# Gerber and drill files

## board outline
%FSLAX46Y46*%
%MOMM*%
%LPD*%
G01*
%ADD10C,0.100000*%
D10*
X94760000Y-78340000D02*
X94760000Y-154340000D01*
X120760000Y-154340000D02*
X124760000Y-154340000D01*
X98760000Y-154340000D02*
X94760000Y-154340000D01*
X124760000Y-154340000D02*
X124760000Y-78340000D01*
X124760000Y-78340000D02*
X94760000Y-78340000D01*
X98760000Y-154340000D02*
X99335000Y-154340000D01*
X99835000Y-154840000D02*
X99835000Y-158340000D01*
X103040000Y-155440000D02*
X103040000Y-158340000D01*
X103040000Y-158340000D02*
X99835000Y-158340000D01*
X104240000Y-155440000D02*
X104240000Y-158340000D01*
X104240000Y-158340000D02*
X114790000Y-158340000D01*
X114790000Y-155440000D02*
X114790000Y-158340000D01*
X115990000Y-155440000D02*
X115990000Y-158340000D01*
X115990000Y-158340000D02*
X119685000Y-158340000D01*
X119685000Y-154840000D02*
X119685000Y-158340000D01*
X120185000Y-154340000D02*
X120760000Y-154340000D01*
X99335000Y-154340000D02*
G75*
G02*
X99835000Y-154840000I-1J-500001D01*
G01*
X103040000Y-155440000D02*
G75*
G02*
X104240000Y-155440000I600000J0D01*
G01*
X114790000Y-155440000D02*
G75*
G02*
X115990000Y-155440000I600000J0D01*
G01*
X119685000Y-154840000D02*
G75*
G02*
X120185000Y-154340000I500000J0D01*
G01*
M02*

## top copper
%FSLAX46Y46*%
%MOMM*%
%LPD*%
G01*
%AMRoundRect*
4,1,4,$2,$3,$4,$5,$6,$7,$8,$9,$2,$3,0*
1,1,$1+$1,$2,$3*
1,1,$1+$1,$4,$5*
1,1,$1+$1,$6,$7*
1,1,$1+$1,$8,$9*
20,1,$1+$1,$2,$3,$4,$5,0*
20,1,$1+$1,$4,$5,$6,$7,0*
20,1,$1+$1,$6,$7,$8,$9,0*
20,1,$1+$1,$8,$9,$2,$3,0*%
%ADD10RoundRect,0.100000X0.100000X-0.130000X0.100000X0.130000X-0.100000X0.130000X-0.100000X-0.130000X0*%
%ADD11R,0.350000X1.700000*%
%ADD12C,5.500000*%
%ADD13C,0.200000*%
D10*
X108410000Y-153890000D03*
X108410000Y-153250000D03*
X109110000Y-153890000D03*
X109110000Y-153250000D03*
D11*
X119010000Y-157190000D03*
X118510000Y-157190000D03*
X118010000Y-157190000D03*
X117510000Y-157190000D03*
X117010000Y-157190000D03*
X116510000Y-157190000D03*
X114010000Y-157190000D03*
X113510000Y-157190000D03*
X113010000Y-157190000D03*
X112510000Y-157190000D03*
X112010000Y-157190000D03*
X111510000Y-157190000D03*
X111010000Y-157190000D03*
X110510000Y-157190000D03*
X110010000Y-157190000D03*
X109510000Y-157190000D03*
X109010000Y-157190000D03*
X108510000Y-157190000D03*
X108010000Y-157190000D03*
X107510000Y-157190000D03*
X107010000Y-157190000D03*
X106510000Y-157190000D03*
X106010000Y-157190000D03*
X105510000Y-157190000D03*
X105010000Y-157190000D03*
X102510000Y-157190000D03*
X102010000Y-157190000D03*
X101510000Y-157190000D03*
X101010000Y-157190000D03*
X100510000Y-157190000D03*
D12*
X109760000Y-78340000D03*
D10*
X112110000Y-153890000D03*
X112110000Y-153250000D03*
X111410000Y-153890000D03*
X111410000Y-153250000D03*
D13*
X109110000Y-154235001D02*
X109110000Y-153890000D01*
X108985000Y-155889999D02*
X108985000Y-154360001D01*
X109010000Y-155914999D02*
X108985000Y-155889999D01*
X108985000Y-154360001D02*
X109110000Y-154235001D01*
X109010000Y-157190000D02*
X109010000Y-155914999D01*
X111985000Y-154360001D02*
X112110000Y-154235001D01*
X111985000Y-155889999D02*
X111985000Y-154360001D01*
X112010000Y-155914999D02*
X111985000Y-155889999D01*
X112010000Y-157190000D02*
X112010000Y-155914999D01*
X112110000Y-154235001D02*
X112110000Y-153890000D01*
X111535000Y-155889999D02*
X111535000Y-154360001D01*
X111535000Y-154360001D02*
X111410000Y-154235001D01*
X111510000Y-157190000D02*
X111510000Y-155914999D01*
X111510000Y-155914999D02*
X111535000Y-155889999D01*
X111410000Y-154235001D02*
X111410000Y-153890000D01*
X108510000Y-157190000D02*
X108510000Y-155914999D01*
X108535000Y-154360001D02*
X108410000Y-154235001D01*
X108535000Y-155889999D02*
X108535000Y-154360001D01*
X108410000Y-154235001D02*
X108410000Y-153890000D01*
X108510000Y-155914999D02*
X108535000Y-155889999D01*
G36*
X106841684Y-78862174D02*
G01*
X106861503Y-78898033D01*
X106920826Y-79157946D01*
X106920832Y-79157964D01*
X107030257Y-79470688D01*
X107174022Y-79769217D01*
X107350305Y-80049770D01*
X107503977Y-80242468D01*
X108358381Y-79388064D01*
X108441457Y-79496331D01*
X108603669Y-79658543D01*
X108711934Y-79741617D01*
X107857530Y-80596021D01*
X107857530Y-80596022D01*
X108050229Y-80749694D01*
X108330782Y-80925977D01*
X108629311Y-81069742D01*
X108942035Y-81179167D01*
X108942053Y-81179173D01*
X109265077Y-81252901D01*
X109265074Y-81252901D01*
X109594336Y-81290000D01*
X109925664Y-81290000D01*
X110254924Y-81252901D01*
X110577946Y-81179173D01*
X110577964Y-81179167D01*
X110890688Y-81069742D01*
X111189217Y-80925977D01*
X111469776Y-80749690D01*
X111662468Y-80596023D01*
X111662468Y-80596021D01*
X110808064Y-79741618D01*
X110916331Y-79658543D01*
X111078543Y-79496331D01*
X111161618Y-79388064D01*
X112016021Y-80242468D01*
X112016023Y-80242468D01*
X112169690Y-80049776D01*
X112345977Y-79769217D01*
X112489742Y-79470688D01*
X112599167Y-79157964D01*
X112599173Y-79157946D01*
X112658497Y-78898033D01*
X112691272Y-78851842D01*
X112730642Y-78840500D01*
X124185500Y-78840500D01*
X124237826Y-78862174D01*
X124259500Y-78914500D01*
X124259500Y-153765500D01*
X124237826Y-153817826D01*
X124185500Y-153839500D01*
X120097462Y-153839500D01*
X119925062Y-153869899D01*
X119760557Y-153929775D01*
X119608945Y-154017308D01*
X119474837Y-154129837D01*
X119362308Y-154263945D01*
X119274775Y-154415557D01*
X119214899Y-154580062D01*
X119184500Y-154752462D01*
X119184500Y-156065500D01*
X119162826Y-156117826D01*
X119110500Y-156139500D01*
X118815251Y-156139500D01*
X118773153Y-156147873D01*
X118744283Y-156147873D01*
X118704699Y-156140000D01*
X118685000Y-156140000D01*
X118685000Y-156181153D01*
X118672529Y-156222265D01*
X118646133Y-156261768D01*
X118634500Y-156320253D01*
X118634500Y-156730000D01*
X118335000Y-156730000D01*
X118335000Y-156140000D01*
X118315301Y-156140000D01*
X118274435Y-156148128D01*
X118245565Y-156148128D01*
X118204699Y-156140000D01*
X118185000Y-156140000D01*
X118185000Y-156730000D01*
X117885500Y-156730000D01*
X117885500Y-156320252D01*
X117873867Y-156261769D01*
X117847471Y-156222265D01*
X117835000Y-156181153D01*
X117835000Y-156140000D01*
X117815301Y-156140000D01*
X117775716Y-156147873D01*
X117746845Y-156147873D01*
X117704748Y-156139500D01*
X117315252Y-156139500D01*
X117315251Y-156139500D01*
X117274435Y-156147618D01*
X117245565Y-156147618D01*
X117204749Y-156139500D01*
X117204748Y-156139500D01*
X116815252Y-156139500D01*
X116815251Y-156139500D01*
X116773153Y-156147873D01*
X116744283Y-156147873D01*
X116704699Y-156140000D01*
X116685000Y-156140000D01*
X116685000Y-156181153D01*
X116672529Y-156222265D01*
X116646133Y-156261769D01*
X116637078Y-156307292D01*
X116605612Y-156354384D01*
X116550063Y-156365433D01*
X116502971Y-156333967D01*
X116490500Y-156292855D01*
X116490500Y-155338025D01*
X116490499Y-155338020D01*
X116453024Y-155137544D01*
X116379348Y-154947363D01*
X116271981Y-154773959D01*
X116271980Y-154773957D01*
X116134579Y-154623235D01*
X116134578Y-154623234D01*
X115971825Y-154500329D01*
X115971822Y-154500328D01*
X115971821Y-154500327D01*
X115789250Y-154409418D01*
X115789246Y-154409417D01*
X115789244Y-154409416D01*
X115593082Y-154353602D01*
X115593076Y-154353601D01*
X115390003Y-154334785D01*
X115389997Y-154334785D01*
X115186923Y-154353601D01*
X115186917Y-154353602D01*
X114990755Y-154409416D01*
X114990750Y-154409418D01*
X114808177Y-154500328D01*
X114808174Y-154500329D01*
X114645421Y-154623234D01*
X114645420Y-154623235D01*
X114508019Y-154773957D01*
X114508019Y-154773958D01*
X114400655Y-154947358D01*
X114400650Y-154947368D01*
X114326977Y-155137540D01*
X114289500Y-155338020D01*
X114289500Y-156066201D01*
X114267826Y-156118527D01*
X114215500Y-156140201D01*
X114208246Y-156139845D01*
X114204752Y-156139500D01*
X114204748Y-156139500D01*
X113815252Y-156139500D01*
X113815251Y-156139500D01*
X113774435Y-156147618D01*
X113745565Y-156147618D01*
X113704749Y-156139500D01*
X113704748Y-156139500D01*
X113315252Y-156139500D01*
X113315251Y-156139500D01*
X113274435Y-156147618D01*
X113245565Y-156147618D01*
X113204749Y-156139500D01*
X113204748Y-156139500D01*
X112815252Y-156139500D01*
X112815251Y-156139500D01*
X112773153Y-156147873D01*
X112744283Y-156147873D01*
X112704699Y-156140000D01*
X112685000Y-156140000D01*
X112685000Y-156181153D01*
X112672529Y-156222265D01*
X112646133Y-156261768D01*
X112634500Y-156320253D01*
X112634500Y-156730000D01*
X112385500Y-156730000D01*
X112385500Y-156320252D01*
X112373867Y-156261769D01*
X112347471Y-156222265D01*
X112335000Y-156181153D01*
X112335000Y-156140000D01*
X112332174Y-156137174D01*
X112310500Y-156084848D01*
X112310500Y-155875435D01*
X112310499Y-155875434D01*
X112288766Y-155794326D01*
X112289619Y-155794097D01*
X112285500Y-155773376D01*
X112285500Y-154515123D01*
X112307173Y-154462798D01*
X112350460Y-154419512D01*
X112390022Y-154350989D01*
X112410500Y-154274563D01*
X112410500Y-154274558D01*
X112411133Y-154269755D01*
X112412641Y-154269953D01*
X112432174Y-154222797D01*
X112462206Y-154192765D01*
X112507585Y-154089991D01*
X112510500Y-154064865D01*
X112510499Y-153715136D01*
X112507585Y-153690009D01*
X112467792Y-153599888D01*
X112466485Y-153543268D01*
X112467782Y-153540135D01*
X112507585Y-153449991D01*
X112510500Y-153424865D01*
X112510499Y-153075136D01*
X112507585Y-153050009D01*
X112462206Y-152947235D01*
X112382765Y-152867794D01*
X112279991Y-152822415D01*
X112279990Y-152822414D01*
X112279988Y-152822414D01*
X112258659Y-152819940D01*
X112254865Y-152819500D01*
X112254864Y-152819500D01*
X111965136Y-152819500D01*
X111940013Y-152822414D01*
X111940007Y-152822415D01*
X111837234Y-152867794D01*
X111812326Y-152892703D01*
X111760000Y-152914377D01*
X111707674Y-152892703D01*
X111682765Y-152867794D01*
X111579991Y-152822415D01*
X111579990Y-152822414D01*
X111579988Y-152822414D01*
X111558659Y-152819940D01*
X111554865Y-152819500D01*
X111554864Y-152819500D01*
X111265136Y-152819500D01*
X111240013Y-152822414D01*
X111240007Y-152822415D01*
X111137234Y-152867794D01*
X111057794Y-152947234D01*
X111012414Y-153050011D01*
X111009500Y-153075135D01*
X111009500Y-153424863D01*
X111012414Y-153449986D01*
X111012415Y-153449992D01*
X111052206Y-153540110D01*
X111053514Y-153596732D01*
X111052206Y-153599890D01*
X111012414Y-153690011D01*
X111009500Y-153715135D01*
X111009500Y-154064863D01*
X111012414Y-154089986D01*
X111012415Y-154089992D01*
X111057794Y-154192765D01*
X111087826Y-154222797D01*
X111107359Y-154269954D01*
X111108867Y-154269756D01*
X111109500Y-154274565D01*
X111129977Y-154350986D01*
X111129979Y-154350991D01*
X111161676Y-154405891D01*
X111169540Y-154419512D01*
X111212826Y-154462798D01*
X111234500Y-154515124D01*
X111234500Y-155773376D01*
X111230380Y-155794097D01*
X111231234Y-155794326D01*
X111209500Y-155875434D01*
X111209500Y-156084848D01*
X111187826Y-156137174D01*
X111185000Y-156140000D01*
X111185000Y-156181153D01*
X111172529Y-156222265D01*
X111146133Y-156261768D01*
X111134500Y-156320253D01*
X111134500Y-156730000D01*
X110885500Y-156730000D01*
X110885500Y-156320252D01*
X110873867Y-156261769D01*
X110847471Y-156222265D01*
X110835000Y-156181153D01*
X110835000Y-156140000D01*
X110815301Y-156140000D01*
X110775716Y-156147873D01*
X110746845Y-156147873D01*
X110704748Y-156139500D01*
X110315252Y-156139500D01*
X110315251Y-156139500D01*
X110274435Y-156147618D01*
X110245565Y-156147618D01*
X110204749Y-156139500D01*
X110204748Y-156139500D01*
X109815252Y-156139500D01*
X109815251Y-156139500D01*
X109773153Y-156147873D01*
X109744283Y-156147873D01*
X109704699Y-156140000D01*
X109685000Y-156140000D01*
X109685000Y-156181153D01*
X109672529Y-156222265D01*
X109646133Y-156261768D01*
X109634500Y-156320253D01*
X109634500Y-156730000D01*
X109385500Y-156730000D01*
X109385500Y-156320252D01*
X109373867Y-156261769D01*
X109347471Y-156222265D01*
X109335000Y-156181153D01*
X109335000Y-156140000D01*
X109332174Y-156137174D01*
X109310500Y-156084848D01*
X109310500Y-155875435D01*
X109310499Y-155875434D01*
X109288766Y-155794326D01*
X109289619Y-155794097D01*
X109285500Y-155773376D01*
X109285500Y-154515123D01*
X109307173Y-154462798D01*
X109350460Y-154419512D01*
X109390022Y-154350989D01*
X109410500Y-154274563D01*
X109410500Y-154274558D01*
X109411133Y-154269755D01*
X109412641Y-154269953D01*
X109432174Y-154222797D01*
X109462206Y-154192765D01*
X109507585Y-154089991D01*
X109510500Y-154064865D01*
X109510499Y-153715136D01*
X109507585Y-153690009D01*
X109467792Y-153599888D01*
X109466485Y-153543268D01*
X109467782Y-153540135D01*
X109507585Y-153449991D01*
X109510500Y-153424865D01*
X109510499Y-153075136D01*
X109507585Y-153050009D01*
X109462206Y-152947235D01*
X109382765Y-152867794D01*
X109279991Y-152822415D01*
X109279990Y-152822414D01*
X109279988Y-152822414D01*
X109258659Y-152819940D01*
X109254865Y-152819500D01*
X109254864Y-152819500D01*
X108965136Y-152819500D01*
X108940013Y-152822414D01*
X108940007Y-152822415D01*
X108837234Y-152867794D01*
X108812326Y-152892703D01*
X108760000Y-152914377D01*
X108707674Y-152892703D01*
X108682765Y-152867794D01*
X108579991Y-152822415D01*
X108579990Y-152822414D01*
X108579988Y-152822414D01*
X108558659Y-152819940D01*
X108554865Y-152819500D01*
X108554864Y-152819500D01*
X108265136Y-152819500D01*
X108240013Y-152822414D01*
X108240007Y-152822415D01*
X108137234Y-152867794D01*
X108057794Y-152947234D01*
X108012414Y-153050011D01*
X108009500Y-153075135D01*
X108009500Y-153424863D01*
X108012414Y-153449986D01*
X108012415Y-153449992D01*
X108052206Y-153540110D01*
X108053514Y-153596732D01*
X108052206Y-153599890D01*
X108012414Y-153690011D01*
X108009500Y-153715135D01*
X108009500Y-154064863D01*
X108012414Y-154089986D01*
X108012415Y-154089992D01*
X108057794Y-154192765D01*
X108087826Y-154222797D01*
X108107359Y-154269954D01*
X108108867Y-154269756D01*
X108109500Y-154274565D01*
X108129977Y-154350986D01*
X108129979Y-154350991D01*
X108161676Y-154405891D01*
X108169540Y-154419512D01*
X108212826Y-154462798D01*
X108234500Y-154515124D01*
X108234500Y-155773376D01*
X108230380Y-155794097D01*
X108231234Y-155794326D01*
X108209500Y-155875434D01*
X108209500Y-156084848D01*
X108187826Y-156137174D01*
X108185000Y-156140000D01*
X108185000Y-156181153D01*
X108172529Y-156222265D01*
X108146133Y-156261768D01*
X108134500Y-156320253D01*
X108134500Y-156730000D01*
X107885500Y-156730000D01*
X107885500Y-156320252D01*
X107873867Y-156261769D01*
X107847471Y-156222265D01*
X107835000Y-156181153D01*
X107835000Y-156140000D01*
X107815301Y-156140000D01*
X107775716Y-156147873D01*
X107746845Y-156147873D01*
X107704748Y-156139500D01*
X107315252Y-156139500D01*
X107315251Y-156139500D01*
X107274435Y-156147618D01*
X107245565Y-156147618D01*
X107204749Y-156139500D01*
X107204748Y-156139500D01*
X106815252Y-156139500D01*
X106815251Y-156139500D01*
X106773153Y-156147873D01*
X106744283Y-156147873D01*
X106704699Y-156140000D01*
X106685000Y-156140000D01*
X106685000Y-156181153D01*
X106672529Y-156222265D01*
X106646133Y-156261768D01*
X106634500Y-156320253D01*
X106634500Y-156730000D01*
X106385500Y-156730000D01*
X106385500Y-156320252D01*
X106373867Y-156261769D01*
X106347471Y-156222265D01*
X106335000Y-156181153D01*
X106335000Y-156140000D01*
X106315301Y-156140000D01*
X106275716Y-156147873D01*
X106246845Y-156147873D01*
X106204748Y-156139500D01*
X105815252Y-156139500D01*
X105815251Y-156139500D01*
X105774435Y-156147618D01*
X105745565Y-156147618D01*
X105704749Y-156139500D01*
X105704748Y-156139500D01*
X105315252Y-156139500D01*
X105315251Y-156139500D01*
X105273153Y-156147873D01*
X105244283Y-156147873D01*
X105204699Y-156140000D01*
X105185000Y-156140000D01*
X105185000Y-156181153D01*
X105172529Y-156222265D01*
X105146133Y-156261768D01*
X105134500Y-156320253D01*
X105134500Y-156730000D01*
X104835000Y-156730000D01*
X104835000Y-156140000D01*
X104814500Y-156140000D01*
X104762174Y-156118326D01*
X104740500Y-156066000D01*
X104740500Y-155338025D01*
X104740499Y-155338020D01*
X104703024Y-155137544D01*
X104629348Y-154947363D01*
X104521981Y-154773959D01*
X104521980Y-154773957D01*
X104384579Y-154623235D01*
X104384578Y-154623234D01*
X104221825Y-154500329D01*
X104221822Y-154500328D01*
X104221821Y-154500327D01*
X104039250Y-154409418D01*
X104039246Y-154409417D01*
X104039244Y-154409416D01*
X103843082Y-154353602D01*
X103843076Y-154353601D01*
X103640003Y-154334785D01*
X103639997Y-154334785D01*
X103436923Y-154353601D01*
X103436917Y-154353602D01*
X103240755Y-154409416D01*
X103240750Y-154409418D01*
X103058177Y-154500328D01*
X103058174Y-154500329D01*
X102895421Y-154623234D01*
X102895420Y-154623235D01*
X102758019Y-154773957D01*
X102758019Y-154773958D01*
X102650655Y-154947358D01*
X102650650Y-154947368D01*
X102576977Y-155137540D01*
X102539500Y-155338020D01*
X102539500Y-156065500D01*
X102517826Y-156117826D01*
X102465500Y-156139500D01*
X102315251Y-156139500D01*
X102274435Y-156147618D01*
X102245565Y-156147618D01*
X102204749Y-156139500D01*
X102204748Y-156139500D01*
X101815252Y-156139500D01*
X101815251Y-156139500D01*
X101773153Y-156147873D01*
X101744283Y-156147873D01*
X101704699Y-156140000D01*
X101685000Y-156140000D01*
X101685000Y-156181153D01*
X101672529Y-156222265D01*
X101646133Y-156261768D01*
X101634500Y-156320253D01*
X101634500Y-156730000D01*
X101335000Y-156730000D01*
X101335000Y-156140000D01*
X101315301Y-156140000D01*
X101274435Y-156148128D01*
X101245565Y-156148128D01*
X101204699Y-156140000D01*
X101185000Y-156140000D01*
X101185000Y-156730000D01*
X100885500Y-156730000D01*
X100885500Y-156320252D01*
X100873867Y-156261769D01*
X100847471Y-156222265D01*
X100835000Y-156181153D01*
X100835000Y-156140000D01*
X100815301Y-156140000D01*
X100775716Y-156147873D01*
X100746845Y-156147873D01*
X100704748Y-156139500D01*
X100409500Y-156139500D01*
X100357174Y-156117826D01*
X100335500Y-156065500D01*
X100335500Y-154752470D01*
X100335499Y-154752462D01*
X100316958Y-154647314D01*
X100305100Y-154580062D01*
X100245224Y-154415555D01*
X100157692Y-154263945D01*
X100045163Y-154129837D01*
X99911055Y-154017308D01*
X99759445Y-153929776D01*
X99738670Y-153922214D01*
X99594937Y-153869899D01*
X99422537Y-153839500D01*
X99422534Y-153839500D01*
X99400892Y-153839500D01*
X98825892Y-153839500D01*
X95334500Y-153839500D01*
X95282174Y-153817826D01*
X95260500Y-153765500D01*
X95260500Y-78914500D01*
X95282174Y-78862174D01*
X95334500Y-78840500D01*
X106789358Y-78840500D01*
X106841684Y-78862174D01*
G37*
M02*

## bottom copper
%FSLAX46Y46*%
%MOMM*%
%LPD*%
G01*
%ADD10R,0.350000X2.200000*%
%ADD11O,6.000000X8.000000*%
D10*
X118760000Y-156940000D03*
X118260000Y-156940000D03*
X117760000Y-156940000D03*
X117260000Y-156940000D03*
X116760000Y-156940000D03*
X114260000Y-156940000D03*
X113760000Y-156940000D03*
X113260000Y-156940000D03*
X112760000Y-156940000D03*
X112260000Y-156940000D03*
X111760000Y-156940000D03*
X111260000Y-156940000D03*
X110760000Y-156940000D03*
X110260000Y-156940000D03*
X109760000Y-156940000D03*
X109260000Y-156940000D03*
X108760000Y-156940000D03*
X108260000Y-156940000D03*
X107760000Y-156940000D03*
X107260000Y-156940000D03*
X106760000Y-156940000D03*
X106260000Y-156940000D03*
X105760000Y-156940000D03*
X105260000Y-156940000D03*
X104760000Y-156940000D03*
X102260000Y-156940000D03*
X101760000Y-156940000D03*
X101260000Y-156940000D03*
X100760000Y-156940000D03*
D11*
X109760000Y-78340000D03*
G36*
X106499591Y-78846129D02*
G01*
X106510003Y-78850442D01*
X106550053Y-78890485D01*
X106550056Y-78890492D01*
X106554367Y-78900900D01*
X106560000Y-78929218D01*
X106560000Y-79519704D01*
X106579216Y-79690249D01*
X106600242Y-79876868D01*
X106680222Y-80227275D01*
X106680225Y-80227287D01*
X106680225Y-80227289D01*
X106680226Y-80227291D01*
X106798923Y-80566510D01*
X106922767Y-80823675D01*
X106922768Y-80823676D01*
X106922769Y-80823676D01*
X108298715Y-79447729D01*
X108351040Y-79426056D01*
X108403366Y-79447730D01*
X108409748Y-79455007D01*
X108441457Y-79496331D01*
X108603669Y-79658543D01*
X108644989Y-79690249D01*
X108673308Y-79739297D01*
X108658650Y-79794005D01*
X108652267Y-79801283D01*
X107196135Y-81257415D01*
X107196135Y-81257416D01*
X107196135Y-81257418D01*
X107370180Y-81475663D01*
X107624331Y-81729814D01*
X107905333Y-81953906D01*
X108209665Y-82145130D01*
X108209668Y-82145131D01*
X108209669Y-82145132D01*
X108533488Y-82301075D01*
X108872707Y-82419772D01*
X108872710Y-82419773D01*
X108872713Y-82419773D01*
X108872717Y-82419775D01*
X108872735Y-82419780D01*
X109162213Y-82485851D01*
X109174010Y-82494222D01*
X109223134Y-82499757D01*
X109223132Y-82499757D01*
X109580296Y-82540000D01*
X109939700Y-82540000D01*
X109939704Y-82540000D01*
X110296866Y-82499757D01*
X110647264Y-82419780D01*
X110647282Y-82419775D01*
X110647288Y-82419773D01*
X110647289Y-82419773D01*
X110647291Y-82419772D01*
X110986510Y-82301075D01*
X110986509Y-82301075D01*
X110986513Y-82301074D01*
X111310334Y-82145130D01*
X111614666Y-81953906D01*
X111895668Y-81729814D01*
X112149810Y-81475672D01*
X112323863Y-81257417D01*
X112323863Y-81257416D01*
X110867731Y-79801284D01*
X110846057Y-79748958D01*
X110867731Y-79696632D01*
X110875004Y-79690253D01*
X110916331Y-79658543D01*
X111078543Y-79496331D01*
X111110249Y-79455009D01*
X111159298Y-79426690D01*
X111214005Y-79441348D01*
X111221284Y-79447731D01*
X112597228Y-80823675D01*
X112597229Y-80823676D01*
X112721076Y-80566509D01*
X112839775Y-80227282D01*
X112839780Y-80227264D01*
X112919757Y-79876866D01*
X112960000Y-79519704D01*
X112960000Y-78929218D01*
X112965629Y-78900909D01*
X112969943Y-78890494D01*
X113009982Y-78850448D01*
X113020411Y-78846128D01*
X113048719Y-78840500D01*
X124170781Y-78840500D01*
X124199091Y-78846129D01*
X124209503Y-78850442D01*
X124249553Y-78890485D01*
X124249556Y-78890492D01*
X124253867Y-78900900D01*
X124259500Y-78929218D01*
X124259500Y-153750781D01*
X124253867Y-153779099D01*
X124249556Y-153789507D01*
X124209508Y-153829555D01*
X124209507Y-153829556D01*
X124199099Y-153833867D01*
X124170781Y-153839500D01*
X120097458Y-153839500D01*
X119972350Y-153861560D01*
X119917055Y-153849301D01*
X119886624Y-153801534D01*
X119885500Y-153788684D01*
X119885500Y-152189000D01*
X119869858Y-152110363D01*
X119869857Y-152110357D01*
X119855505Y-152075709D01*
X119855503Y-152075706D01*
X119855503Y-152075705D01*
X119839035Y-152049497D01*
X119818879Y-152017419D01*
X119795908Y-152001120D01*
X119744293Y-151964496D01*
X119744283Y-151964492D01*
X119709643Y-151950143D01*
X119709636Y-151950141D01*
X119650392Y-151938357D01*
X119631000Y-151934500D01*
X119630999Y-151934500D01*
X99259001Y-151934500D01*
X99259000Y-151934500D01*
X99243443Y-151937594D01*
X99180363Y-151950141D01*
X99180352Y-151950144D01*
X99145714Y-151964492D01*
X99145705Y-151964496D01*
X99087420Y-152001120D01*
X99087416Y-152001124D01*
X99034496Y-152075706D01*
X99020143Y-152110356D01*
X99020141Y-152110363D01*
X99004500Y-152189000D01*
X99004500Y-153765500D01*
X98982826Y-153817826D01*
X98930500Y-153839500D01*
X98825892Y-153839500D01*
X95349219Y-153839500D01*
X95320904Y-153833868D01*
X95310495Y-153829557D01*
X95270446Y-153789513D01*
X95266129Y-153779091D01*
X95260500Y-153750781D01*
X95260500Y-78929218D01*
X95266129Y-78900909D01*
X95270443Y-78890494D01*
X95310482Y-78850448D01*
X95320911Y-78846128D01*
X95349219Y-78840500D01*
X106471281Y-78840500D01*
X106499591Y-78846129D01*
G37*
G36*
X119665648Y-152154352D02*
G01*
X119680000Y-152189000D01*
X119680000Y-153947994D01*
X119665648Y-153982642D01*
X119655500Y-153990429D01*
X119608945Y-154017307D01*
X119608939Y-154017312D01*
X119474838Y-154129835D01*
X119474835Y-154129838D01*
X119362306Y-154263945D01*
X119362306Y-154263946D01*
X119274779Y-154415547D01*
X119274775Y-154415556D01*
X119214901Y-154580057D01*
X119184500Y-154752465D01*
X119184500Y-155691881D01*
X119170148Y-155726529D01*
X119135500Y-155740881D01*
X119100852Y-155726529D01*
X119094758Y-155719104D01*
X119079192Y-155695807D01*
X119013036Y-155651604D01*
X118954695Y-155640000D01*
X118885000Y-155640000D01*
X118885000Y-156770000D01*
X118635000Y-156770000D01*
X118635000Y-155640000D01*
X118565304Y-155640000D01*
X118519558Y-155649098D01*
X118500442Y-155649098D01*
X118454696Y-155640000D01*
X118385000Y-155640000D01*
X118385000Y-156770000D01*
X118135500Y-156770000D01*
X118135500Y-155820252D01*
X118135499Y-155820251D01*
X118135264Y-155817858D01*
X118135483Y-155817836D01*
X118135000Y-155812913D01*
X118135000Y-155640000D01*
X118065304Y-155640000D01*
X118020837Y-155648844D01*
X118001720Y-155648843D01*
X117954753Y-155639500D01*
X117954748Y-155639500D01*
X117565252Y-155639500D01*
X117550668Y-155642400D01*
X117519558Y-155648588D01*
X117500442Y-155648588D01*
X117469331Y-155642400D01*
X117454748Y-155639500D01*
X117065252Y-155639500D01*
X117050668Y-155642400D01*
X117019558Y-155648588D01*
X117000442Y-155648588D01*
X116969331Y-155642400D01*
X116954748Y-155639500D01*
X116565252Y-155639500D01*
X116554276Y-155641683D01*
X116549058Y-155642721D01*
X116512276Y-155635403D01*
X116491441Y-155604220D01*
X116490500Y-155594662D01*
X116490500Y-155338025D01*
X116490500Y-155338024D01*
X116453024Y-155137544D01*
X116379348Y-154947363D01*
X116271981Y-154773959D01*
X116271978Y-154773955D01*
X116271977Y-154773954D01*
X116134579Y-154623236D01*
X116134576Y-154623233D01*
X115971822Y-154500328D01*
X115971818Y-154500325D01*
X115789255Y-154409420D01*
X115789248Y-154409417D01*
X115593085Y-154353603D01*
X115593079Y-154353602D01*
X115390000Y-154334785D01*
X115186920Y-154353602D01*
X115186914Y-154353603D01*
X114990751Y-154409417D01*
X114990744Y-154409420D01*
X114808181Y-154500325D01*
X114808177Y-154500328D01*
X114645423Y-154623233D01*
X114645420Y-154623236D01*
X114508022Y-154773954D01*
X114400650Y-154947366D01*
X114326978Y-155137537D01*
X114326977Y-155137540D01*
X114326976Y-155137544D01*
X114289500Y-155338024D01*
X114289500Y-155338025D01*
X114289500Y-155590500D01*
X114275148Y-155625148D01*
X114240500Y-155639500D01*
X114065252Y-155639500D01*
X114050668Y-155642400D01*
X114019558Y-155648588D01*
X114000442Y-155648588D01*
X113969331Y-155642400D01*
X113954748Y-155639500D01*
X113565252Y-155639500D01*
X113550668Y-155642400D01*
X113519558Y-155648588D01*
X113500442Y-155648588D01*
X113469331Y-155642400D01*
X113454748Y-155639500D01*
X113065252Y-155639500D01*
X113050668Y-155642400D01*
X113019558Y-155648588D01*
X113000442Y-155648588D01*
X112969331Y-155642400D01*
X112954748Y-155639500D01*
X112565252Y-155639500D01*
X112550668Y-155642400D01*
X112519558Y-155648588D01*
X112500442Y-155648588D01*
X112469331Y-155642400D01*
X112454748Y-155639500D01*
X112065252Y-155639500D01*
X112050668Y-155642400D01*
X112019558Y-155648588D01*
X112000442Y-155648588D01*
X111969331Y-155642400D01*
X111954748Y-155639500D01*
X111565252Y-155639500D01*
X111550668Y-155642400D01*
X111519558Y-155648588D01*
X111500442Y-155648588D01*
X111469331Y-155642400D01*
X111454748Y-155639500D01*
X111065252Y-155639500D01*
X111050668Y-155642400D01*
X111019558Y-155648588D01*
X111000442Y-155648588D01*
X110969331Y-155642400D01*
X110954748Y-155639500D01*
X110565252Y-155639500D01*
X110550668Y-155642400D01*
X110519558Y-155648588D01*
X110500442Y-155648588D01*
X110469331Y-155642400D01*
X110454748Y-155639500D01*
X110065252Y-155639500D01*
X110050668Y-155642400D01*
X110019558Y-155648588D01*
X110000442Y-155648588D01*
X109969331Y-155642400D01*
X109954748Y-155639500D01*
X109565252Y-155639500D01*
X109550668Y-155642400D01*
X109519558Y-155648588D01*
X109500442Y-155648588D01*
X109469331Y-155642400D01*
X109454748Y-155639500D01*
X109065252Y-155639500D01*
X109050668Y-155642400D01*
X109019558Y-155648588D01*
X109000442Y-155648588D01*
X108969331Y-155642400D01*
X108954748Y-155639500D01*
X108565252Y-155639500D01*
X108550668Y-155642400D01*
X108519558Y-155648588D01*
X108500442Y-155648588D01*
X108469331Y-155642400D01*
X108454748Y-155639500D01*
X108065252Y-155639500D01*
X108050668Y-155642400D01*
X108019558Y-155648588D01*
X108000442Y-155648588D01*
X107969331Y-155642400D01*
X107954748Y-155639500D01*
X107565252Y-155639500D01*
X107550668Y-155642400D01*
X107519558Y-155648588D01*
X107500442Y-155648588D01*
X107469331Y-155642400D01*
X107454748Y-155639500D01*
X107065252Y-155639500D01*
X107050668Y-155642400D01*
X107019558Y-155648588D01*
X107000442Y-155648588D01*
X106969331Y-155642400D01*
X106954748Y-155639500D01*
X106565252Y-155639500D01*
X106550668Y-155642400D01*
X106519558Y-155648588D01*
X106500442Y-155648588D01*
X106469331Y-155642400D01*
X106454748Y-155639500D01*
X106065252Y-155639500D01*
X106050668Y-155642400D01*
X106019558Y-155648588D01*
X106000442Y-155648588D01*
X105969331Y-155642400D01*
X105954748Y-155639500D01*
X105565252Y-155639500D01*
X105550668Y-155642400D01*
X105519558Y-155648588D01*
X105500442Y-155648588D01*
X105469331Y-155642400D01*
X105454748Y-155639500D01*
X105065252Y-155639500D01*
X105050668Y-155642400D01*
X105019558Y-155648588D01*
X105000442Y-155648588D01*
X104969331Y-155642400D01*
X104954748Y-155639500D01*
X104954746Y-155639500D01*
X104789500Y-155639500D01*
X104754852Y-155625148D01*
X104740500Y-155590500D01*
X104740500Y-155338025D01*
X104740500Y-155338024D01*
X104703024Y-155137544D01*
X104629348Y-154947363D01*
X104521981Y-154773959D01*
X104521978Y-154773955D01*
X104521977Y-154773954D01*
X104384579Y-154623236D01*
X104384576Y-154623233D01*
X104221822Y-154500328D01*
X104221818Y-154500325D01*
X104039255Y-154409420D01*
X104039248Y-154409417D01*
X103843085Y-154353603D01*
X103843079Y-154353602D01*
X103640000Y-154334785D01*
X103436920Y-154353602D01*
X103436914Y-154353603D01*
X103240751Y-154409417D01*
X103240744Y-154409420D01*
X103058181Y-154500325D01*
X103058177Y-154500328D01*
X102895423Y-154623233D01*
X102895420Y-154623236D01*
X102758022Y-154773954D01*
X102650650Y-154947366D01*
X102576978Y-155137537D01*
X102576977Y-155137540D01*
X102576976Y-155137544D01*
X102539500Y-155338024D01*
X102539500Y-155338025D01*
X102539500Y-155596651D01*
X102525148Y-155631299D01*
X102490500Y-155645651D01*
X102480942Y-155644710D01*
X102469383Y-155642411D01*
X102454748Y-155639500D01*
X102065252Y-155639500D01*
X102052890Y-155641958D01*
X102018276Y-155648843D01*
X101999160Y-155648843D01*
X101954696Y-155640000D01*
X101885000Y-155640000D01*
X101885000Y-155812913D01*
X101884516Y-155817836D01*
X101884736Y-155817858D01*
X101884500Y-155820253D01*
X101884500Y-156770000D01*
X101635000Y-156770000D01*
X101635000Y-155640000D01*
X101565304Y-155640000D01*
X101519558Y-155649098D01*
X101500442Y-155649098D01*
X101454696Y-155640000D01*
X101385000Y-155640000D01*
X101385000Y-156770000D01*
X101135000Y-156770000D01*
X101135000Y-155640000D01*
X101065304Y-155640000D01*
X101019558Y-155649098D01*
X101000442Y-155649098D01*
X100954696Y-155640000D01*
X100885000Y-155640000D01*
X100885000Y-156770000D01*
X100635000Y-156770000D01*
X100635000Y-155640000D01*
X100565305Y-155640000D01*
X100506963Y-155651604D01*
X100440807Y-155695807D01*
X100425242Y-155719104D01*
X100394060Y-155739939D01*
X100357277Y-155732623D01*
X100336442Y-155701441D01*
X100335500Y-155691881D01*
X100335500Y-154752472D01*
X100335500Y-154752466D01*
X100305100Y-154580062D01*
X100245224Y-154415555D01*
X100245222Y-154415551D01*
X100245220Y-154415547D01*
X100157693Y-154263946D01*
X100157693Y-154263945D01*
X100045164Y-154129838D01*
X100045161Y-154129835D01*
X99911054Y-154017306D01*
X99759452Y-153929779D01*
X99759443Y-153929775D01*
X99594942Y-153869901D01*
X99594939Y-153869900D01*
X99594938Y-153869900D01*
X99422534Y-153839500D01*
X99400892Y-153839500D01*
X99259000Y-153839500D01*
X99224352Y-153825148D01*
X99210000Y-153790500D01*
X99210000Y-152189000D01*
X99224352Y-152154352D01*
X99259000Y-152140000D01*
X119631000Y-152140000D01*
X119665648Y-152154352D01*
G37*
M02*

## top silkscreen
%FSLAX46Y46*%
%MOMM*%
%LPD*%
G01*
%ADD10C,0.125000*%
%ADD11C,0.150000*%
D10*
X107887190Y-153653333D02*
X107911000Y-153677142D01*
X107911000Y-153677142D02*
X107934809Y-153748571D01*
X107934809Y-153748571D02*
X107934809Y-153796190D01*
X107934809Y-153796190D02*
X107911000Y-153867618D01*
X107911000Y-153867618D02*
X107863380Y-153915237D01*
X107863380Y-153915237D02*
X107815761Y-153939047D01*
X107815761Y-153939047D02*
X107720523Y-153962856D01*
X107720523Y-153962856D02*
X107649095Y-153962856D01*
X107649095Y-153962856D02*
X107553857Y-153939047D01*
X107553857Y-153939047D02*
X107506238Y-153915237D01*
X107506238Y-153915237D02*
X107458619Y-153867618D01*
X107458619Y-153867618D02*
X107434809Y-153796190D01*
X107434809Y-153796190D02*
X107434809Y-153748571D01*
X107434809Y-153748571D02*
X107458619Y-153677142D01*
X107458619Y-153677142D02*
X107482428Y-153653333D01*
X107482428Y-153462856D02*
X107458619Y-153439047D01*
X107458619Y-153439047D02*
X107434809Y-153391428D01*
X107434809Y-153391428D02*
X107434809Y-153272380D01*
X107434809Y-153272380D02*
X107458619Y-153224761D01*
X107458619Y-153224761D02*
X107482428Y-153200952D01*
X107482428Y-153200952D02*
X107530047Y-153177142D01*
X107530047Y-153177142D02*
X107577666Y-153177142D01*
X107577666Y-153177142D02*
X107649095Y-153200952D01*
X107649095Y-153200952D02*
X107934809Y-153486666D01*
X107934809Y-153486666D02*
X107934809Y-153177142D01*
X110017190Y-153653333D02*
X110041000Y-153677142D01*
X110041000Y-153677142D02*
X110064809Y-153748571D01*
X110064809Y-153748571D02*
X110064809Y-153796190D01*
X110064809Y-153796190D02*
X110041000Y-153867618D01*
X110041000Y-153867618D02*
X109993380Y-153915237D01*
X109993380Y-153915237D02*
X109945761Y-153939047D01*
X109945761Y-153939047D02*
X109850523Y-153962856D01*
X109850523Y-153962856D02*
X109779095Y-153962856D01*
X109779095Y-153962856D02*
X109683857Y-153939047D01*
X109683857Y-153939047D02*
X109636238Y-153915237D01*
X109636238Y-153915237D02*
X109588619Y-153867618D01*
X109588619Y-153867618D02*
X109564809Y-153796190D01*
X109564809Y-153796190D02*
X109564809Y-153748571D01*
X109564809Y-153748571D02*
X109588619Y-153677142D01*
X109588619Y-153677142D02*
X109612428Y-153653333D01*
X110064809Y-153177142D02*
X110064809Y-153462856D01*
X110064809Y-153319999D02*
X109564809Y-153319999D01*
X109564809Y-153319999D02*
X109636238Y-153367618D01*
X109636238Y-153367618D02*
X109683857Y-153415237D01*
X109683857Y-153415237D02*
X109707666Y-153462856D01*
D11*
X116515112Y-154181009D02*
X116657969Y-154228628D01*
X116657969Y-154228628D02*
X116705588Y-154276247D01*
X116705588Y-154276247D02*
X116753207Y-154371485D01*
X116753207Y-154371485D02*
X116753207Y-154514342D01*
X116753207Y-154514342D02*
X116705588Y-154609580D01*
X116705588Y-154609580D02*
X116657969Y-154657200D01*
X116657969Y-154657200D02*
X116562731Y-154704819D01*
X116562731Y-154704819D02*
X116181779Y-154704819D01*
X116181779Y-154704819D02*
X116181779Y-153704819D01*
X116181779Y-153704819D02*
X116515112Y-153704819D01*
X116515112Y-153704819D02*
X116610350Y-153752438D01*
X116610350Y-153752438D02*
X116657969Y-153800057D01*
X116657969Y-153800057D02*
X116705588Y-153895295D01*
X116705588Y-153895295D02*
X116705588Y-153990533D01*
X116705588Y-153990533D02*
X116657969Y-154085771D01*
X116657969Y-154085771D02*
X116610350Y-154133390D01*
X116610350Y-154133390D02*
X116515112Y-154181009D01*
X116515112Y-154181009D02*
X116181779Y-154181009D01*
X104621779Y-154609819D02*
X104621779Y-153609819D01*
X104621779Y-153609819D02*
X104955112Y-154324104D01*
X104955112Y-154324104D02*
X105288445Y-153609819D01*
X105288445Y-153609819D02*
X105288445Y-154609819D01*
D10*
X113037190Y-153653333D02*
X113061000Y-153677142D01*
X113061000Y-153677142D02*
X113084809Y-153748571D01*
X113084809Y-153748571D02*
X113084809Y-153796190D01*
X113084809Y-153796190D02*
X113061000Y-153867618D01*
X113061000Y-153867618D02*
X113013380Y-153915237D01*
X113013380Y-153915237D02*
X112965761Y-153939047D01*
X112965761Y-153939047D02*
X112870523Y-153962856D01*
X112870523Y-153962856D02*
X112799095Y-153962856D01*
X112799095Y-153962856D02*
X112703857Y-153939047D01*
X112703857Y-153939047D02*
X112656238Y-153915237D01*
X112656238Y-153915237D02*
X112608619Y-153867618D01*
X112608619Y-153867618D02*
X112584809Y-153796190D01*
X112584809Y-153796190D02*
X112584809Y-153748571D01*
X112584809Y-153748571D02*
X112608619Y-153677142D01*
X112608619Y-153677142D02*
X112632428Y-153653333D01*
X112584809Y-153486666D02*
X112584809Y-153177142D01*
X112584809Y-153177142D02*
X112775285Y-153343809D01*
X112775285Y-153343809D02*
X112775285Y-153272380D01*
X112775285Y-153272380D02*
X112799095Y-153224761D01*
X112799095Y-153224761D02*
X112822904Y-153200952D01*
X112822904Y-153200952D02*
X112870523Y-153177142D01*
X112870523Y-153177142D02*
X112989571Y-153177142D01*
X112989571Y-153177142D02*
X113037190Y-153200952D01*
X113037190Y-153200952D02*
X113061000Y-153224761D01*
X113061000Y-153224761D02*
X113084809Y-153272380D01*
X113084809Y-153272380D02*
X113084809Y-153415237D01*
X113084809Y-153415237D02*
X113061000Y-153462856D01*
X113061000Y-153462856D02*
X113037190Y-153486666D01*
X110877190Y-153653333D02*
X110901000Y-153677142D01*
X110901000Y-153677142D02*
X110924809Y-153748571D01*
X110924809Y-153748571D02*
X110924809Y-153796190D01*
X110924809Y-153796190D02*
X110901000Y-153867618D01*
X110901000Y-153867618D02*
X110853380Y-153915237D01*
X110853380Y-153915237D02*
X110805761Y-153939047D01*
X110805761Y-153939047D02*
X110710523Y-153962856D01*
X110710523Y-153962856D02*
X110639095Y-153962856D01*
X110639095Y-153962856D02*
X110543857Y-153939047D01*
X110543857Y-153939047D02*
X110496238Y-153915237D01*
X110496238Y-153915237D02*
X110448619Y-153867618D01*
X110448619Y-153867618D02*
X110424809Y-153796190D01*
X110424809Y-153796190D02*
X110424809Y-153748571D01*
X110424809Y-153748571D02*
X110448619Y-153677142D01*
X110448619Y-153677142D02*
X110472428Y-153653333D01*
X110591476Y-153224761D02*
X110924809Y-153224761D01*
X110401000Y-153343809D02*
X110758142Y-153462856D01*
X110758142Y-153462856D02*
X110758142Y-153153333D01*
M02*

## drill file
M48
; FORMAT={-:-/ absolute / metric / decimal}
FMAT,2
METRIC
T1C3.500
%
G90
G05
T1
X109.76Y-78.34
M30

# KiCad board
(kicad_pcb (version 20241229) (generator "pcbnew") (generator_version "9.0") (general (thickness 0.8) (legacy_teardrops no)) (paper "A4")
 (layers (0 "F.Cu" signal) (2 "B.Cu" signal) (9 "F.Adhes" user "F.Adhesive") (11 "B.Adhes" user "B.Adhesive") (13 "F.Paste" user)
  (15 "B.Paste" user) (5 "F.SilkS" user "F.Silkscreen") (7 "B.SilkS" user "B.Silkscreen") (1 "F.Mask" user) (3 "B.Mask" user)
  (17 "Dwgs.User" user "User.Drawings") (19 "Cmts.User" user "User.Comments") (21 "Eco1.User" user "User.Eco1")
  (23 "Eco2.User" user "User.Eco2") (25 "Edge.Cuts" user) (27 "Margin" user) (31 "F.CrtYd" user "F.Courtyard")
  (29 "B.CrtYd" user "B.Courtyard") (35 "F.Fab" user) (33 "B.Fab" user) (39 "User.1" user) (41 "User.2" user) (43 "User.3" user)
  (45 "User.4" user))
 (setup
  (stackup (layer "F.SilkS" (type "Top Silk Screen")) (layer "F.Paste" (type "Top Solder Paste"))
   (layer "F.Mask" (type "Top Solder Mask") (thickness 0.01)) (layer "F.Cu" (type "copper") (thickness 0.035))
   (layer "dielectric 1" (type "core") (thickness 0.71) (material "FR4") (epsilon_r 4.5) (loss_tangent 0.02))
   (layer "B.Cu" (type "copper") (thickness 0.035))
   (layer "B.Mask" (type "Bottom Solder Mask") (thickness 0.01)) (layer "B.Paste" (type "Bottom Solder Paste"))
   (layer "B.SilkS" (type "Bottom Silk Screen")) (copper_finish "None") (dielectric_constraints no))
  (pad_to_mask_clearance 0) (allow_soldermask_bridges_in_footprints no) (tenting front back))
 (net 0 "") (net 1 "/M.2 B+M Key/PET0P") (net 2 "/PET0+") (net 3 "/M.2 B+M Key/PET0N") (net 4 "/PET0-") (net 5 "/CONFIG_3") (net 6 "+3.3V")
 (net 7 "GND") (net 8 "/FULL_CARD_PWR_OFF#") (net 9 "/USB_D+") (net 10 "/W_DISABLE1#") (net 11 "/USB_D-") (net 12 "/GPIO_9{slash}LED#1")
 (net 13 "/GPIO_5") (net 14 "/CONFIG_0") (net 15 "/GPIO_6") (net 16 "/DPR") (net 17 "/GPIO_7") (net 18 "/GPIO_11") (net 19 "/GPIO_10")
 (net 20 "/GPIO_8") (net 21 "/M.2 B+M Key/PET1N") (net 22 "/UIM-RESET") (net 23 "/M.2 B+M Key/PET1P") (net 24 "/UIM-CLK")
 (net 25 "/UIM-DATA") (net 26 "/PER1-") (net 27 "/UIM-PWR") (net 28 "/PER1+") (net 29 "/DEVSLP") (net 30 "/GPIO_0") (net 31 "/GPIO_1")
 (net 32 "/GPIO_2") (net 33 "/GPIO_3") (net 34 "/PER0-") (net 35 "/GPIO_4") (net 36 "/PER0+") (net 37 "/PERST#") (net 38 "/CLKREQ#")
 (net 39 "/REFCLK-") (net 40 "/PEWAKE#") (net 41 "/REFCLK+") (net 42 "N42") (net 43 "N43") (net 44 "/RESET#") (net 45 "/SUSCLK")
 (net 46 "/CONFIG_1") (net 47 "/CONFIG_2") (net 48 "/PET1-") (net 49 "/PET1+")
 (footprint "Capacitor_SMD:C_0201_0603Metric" (layer "F.Cu") (at 108.41 153.57 90)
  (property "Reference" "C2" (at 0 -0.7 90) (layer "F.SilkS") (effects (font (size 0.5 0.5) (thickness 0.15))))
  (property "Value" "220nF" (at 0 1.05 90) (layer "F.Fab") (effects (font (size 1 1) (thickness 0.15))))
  (pad "" smd roundrect (at -0.345 0 90) (size 0.318 0.36) (layers "F.Paste") (roundrect_rratio 0.25))
  (pad "" smd roundrect (at 0.345 0 90) (size 0.318 0.36) (layers "F.Paste") (roundrect_rratio 0.25))
  (pad "1" smd roundrect (at -0.32 0 90) (size 0.46 0.4) (layers "F.Cu" "F.Mask") (roundrect_rratio 0.25) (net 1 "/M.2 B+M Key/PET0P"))
  (pad "2" smd roundrect (at 0.32 0 90) (size 0.46 0.4) (layers "F.Cu" "F.Mask") (roundrect_rratio 0.25) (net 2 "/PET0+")))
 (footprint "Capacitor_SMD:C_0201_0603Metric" (layer "F.Cu") (at 109.11 153.57 90)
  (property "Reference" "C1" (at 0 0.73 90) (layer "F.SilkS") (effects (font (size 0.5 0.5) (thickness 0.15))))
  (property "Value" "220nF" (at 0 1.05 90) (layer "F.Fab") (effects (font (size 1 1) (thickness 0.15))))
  (pad "" smd roundrect (at -0.345 0 90) (size 0.318 0.36) (layers "F.Paste") (roundrect_rratio 0.25))
  (pad "" smd roundrect (at 0.345 0 90) (size 0.318 0.36) (layers "F.Paste") (roundrect_rratio 0.25))
  (pad "1" smd roundrect (at -0.32 0 90) (size 0.46 0.4) (layers "F.Cu" "F.Mask") (roundrect_rratio 0.25) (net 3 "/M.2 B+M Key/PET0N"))
  (pad "2" smd roundrect (at 0.32 0 90) (size 0.46 0.4) (layers "F.Cu" "F.Mask") (roundrect_rratio 0.25) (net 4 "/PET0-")))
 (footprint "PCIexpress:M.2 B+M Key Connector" (layer "F.Cu") (at 109.76 157.23)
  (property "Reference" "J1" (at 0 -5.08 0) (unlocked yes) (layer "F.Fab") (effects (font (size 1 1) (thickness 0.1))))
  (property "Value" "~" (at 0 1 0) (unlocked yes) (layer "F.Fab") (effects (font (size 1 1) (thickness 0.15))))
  (fp_line (start -11 -2.89) (end -10.425 -2.89) (stroke (width 0.1) (type default)) (layer "Edge.Cuts"))
  (fp_line (start -9.925 -2.39) (end -9.925 1.11) (stroke (width 0.1) (type default)) (layer "Edge.Cuts"))
  (fp_line (start -6.72 -1.79) (end -6.72 1.11) (stroke (width 0.1) (type default)) (layer "Edge.Cuts"))
  (fp_line (start -6.72 1.11) (end -9.925 1.11) (stroke (width 0.1) (type default)) (layer "Edge.Cuts"))
  (fp_line (start -5.52 -1.79) (end -5.52 1.11) (stroke (width 0.1) (type default)) (layer "Edge.Cuts"))
  (fp_line (start -5.52 1.11) (end 5.03 1.11) (stroke (width 0.1) (type default)) (layer "Edge.Cuts"))
  (fp_line (start 5.03 -1.79) (end 5.03 1.11) (stroke (width 0.1) (type default)) (layer "Edge.Cuts"))
  (fp_line (start 6.23 -1.79) (end 6.23 1.11) (stroke (width 0.1) (type default)) (layer "Edge.Cuts"))
  (fp_line (start 6.23 1.11) (end 9.925 1.11) (stroke (width 0.1) (type default)) (layer "Edge.Cuts"))
  (fp_line (start 9.925 -2.39) (end 9.925 1.11) (stroke (width 0.1) (type default)) (layer "Edge.Cuts"))
  (fp_line (start 10.425 -2.89) (end 11 -2.89) (stroke (width 0.1) (type default)) (layer "Edge.Cuts"))
  (fp_arc (start -10.425 -2.89) (mid -10.071447 -2.743553) (end -9.925 -2.39) (stroke (width 0.1) (type default)) (layer "Edge.Cuts"))
  (fp_arc (start -6.72 -1.79) (mid -6.12 -2.39) (end -5.52 -1.79) (stroke (width 0.1) (type default)) (layer "Edge.Cuts"))
  (fp_arc (start 5.03 -1.79) (mid 5.63 -2.39) (end 6.23 -1.79) (stroke (width 0.1) (type default)) (layer "Edge.Cuts"))
  (fp_arc (start 9.925 -2.39) (mid 10.071447 -2.743553) (end 10.425 -2.89) (stroke (width 0.1) (type default)) (layer "Edge.Cuts"))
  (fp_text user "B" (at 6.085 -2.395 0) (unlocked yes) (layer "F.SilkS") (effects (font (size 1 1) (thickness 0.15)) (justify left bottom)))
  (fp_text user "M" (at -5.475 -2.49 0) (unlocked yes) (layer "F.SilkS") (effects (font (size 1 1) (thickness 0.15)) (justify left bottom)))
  (pad "1" smd rect (at 9.25 -0.04 180) (size 0.35 1.7) (layers "F.Cu") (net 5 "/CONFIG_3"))
  (pad "2" smd rect (at 9 -0.29 180) (size 0.35 2.2) (layers "B.Cu") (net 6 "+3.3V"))
  (pad "3" smd rect (at 8.75 -0.04 180) (size 0.35 1.7) (layers "F.Cu") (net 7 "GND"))
  (pad "4" smd rect (at 8.5 -0.29 180) (size 0.35 2.2) (layers "B.Cu") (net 6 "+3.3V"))
  (pad "5" smd rect (at 8.25 -0.04 180) (size 0.35 1.7) (layers "F.Cu") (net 7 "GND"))
  (pad "6" smd rect (at 8 -0.29 180) (size 0.35 2.2) (layers "B.Cu") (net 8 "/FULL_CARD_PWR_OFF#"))
  (pad "7" smd rect (at 7.75 -0.04 180) (size 0.35 1.7) (layers "F.Cu") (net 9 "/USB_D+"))
  (pad "8" smd rect (at 7.5 -0.29 180) (size 0.35 2.2) (layers "B.Cu") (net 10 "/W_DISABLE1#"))
  (pad "9" smd rect (at 7.25 -0.04 180) (size 0.35 1.7) (layers "F.Cu") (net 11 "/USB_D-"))
  (pad "10" smd rect (at 7 -0.29 180) (size 0.35 2.2) (layers "B.Cu") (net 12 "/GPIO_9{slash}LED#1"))
  (pad "11" smd rect (at 6.75 -0.04 180) (size 0.35 1.7) (layers "F.Cu") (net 7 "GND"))
  (pad "20" smd rect (at 4.5 -0.29 180) (size 0.35 2.2) (layers "B.Cu") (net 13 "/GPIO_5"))
  (pad "21" smd rect (at 4.25 -0.04 180) (size 0.35 1.7) (layers "F.Cu") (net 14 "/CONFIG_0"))
  (pad "22" smd rect (at 4 -0.29 180) (size 0.35 2.2) (layers "B.Cu") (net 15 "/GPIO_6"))
  (pad "23" smd rect (at 3.75 -0.04 180) (size 0.35 1.7) (layers "F.Cu") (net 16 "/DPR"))
  (pad "24" smd rect (at 3.5 -0.29 180) (size 0.35 2.2) (layers "B.Cu") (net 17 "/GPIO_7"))
  (pad "25" smd rect (at 3.25 -0.04 180) (size 0.35 1.7) (layers "F.Cu") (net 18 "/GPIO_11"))
  (pad "26" smd rect (at 3 -0.29 180) (size 0.35 2.2) (layers "B.Cu") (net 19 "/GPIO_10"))
  (pad "27" smd rect (at 2.75 -0.04 180) (size 0.35 1.7) (layers "F.Cu") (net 7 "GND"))
  (pad "28" smd rect (at 2.5 -0.29 180) (size 0.35 2.2) (layers "B.Cu") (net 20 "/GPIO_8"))
  (pad "29" smd rect (at 2.25 -0.04 180) (size 0.35 1.7) (layers "F.Cu") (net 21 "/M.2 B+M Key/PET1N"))
  (pad "30" smd rect (at 2 -0.29 180) (size 0.35 2.2) (layers "B.Cu") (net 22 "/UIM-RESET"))
  (pad "31" smd rect (at 1.75 -0.04 180) (size 0.35 1.7) (layers "F.Cu") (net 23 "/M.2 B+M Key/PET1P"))
  (pad "32" smd rect (at 1.5 -0.29 180) (size 0.35 2.2) (layers "B.Cu") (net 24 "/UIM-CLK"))
  (pad "33" smd rect (at 1.25 -0.04 180) (size 0.35 1.7) (layers "F.Cu") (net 7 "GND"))
  (pad "34" smd rect (at 1 -0.29 180) (size 0.35 2.2) (layers "B.Cu") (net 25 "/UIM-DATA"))
  (pad "35" smd rect (at 0.75 -0.04 180) (size 0.35 1.7) (layers "F.Cu") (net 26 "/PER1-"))
  (pad "36" smd rect (at 0.5 -0.29 180) (size 0.35 2.2) (layers "B.Cu") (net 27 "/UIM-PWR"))
  (pad "37" smd rect (at 0.25 -0.04 180) (size 0.35 1.7) (layers "F.Cu") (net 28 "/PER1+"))
  (pad "38" smd rect (at 0 -0.29 180) (size 0.35 2.2) (layers "B.Cu") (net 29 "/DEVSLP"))
  (pad "39" smd rect (at -0.25 -0.04 180) (size 0.35 1.7) (layers "F.Cu") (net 7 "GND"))
  (pad "40" smd rect (at -0.5 -0.29 180) (size 0.35 2.2) (layers "B.Cu") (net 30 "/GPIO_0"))
  (pad "41" smd rect (at -0.75 -0.04 180) (size 0.35 1.7) (layers "F.Cu") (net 3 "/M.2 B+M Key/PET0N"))
  (pad "42" smd rect (at -1 -0.29 180) (size 0.35 2.2) (layers "B.Cu") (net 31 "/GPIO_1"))
  (pad "43" smd rect (at -1.25 -0.04 180) (size 0.35 1.7) (layers "F.Cu") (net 1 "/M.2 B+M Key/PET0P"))
  (pad "44" smd rect (at -1.5 -0.29 180) (size 0.35 2.2) (layers "B.Cu") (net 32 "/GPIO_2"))
  (pad "45" smd rect (at -1.75 -0.04 180) (size 0.35 1.7) (layers "F.Cu") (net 7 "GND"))
  (pad "46" smd rect (at -2 -0.29 180) (size 0.35 2.2) (layers "B.Cu") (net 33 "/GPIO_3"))
  (pad "47" smd rect (at -2.25 -0.04 180) (size 0.35 1.7) (layers "F.Cu") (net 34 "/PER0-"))
  (pad "48" smd rect (at -2.5 -0.29 180) (size 0.35 2.2) (layers "B.Cu") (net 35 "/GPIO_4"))
  (pad "49" smd rect (at -2.75 -0.04 180) (size 0.35 1.7) (layers "F.Cu") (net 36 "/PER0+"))
  (pad "50" smd rect (at -3 -0.29 180) (size 0.35 2.2) (layers "B.Cu") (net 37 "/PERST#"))
  (pad "51" smd rect (at -3.25 -0.04 180) (size 0.35 1.7) (layers "F.Cu") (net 7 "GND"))
  (pad "52" smd rect (at -3.5 -0.29 180) (size 0.35 2.2) (layers "B.Cu") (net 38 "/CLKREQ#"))
  (pad "53" smd rect (at -3.75 -0.04 180) (size 0.35 1.7) (layers "F.Cu") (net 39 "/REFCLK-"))
  (pad "54" smd rect (at -4 -0.29 180) (size 0.35 2.2) (layers "B.Cu") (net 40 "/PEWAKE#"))
  (pad "55" smd rect (at -4.25 -0.04 180) (size 0.35 1.7) (layers "F.Cu") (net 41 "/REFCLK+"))
  (pad "56" smd rect (at -4.5 -0.29 180) (size 0.35 2.2) (layers "B.Cu") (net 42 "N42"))
  (pad "57" smd rect (at -4.75 -0.04 180) (size 0.35 1.7) (layers "F.Cu") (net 7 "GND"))
  (pad "58" smd rect (at -5 -0.29 180) (size 0.35 2.2) (layers "B.Cu") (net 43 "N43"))
  (pad "67" smd rect (at -7.25 -0.04 180) (size 0.35 1.7) (layers "F.Cu") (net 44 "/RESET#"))
  (pad "68" smd rect (at -7.5 -0.29 180) (size 0.35 2.2) (layers "B.Cu") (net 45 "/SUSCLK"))
  (pad "69" smd rect (at -7.75 -0.04 180) (size 0.35 1.7) (layers "F.Cu") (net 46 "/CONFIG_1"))
  (pad "70" smd rect (at -8 -0.29 180) (size 0.35 2.2) (layers "B.Cu") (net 6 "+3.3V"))
  (pad "71" smd rect (at -8.25 -0.04 180) (size 0.35 1.7) (layers "F.Cu") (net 7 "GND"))
  (pad "72" smd rect (at -8.5 -0.29 180) (size 0.35 2.2) (layers "B.Cu") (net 6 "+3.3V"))
  (pad "73" smd rect (at -8.75 -0.04 180) (size 0.35 1.7) (layers "F.Cu") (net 7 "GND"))
  (pad "74" smd rect (at -9 -0.29 180) (size 0.35 2.2) (layers "B.Cu") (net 6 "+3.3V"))
  (pad "75" smd rect (at -9.25 -0.04 180) (size 0.35 1.7) (layers "F.Cu") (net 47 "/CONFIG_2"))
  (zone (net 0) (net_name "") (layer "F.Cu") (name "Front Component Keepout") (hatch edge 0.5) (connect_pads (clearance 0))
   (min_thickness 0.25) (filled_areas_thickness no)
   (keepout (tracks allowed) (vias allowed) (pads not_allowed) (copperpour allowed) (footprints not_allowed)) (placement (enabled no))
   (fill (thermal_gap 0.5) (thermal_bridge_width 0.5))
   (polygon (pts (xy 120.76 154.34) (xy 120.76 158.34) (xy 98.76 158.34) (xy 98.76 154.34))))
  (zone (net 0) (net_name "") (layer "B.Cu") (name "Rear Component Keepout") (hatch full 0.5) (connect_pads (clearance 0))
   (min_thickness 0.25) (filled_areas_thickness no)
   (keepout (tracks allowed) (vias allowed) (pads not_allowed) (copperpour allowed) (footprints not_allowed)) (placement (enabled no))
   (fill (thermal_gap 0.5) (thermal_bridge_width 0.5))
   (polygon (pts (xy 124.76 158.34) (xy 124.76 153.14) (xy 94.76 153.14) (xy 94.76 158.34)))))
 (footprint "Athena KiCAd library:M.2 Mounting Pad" (layer "F.Cu") (at 109.76 78.34)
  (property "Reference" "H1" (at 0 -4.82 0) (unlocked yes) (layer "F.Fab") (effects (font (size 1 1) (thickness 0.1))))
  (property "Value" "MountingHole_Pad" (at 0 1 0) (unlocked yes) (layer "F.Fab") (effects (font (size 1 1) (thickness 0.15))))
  (pad "1" thru_hole circle (at 0 0) (size 5.5 5.5) (drill 3.5) (layers "*.Cu" "*.Mask") (remove_unused_layers no) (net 7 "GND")
   (padstack (mode front_inner_back)
    (layer "Inner" (shape circle) (size 5.5 5.5) (zone_connect -1))
    (layer "B.Cu" (shape oval) (size 6 8) (thermal_bridge_angle 45) (zone_connect -1)))))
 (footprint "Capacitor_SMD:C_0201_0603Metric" (layer "F.Cu") (at 112.11 153.57 90)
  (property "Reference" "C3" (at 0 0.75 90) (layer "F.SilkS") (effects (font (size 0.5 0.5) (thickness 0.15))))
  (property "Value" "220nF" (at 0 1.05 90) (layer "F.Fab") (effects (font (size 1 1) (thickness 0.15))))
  (pad "" smd roundrect (at -0.345 0 90) (size 0.318 0.36) (layers "F.Paste") (roundrect_rratio 0.25))
  (pad "" smd roundrect (at 0.345 0 90) (size 0.318 0.36) (layers "F.Paste") (roundrect_rratio 0.25))
  (pad "1" smd roundrect (at -0.32 0 90) (size 0.46 0.4) (layers "F.Cu" "F.Mask") (roundrect_rratio 0.25) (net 21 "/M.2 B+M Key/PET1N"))
  (pad "2" smd roundrect (at 0.32 0 90) (size 0.46 0.4) (layers "F.Cu" "F.Mask") (roundrect_rratio 0.25) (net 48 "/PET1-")))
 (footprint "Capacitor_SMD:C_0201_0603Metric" (layer "F.Cu") (at 111.41 153.57 90)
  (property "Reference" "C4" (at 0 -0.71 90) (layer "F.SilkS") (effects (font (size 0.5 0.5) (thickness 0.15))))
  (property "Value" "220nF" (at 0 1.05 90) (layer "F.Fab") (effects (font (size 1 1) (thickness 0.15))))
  (pad "" smd roundrect (at -0.345 0 90) (size 0.318 0.36) (layers "F.Paste") (roundrect_rratio 0.25))
  (pad "" smd roundrect (at 0.345 0 90) (size 0.318 0.36) (layers "F.Paste") (roundrect_rratio 0.25))
  (pad "1" smd roundrect (at -0.32 0 90) (size 0.46 0.4) (layers "F.Cu" "F.Mask") (roundrect_rratio 0.25) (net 23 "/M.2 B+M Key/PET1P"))
  (pad "2" smd roundrect (at 0.32 0 90) (size 0.46 0.4) (layers "F.Cu" "F.Mask") (roundrect_rratio 0.25) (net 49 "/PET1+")))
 (gr_line (start 94.76 78.34) (end 94.76 154.34) (stroke (width 0.1) (type default)) (layer "Edge.Cuts"))
 (gr_line (start 120.76 154.34) (end 124.76 154.34) (stroke (width 0.1) (type default)) (layer "Edge.Cuts"))
 (gr_line (start 98.76 154.34) (end 94.76 154.34) (stroke (width 0.1) (type default)) (layer "Edge.Cuts"))
 (gr_line (start 124.76 154.34) (end 124.76 78.34) (stroke (width 0.1) (type default)) (layer "Edge.Cuts"))
 (gr_line (start 124.76 78.34) (end 94.76 78.34) (stroke (width 0.1) (type default)) (layer "Edge.Cuts"))
 (segment (start 109.11 154.235001) (end 109.11 153.89) (width 0.2) (layer "F.Cu") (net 3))
 (segment (start 108.985 155.889999) (end 108.985 154.360001) (width 0.2) (layer "F.Cu") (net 3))
 (segment (start 109.01 155.914999) (end 108.985 155.889999) (width 0.2) (layer "F.Cu") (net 3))
 (segment (start 108.985 154.360001) (end 109.11 154.235001) (width 0.2) (layer "F.Cu") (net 3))
 (segment (start 109.01 157.19) (end 109.01 155.914999) (width 0.2) (layer "F.Cu") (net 3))
 (segment (start 111.985 154.360001) (end 112.11 154.235001) (width 0.2) (layer "F.Cu") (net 21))
 (segment (start 111.985 155.889999) (end 111.985 154.360001) (width 0.2) (layer "F.Cu") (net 21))
 (segment (start 112.01 155.914999) (end 111.985 155.889999) (width 0.2) (layer "F.Cu") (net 21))
 (segment (start 112.01 157.19) (end 112.01 155.914999) (width 0.2) (layer "F.Cu") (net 21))
 (segment (start 112.11 154.235001) (end 112.11 153.89) (width 0.2) (layer "F.Cu") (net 21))
 (segment (start 111.535 155.889999) (end 111.535 154.360001) (width 0.2) (layer "F.Cu") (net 23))
 (segment (start 111.535 154.360001) (end 111.41 154.235001) (width 0.2) (layer "F.Cu") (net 23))
 (segment (start 111.51 157.19) (end 111.51 155.914999) (width 0.2) (layer "F.Cu") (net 23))
 (segment (start 111.51 155.914999) (end 111.535 155.889999) (width 0.2) (layer "F.Cu") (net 23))
 (segment (start 111.41 154.235001) (end 111.41 153.89) (width 0.2) (layer "F.Cu") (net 23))
 (segment (start 108.51 157.19) (end 108.51 155.914999) (width 0.2) (layer "F.Cu") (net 1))
 (segment (start 108.535 154.360001) (end 108.41 154.235001) (width 0.2) (layer "F.Cu") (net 1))
 (segment (start 108.535 155.889999) (end 108.535 154.360001) (width 0.2) (layer "F.Cu") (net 1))
 (segment (start 108.41 154.235001) (end 108.41 153.89) (width 0.2) (layer "F.Cu") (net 1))
 (segment (start 108.51 155.914999) (end 108.535 155.889999) (width 0.2) (layer "F.Cu") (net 1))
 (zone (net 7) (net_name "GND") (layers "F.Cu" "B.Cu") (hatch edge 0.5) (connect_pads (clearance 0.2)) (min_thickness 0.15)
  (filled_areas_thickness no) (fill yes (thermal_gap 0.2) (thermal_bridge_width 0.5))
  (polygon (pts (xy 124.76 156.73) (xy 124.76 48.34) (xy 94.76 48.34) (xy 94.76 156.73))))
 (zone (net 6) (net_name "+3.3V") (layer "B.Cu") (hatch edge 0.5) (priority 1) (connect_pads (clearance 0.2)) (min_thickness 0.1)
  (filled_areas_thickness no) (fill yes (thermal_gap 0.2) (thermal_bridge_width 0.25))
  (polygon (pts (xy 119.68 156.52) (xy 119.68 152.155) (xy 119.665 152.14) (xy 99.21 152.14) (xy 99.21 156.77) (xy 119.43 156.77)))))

